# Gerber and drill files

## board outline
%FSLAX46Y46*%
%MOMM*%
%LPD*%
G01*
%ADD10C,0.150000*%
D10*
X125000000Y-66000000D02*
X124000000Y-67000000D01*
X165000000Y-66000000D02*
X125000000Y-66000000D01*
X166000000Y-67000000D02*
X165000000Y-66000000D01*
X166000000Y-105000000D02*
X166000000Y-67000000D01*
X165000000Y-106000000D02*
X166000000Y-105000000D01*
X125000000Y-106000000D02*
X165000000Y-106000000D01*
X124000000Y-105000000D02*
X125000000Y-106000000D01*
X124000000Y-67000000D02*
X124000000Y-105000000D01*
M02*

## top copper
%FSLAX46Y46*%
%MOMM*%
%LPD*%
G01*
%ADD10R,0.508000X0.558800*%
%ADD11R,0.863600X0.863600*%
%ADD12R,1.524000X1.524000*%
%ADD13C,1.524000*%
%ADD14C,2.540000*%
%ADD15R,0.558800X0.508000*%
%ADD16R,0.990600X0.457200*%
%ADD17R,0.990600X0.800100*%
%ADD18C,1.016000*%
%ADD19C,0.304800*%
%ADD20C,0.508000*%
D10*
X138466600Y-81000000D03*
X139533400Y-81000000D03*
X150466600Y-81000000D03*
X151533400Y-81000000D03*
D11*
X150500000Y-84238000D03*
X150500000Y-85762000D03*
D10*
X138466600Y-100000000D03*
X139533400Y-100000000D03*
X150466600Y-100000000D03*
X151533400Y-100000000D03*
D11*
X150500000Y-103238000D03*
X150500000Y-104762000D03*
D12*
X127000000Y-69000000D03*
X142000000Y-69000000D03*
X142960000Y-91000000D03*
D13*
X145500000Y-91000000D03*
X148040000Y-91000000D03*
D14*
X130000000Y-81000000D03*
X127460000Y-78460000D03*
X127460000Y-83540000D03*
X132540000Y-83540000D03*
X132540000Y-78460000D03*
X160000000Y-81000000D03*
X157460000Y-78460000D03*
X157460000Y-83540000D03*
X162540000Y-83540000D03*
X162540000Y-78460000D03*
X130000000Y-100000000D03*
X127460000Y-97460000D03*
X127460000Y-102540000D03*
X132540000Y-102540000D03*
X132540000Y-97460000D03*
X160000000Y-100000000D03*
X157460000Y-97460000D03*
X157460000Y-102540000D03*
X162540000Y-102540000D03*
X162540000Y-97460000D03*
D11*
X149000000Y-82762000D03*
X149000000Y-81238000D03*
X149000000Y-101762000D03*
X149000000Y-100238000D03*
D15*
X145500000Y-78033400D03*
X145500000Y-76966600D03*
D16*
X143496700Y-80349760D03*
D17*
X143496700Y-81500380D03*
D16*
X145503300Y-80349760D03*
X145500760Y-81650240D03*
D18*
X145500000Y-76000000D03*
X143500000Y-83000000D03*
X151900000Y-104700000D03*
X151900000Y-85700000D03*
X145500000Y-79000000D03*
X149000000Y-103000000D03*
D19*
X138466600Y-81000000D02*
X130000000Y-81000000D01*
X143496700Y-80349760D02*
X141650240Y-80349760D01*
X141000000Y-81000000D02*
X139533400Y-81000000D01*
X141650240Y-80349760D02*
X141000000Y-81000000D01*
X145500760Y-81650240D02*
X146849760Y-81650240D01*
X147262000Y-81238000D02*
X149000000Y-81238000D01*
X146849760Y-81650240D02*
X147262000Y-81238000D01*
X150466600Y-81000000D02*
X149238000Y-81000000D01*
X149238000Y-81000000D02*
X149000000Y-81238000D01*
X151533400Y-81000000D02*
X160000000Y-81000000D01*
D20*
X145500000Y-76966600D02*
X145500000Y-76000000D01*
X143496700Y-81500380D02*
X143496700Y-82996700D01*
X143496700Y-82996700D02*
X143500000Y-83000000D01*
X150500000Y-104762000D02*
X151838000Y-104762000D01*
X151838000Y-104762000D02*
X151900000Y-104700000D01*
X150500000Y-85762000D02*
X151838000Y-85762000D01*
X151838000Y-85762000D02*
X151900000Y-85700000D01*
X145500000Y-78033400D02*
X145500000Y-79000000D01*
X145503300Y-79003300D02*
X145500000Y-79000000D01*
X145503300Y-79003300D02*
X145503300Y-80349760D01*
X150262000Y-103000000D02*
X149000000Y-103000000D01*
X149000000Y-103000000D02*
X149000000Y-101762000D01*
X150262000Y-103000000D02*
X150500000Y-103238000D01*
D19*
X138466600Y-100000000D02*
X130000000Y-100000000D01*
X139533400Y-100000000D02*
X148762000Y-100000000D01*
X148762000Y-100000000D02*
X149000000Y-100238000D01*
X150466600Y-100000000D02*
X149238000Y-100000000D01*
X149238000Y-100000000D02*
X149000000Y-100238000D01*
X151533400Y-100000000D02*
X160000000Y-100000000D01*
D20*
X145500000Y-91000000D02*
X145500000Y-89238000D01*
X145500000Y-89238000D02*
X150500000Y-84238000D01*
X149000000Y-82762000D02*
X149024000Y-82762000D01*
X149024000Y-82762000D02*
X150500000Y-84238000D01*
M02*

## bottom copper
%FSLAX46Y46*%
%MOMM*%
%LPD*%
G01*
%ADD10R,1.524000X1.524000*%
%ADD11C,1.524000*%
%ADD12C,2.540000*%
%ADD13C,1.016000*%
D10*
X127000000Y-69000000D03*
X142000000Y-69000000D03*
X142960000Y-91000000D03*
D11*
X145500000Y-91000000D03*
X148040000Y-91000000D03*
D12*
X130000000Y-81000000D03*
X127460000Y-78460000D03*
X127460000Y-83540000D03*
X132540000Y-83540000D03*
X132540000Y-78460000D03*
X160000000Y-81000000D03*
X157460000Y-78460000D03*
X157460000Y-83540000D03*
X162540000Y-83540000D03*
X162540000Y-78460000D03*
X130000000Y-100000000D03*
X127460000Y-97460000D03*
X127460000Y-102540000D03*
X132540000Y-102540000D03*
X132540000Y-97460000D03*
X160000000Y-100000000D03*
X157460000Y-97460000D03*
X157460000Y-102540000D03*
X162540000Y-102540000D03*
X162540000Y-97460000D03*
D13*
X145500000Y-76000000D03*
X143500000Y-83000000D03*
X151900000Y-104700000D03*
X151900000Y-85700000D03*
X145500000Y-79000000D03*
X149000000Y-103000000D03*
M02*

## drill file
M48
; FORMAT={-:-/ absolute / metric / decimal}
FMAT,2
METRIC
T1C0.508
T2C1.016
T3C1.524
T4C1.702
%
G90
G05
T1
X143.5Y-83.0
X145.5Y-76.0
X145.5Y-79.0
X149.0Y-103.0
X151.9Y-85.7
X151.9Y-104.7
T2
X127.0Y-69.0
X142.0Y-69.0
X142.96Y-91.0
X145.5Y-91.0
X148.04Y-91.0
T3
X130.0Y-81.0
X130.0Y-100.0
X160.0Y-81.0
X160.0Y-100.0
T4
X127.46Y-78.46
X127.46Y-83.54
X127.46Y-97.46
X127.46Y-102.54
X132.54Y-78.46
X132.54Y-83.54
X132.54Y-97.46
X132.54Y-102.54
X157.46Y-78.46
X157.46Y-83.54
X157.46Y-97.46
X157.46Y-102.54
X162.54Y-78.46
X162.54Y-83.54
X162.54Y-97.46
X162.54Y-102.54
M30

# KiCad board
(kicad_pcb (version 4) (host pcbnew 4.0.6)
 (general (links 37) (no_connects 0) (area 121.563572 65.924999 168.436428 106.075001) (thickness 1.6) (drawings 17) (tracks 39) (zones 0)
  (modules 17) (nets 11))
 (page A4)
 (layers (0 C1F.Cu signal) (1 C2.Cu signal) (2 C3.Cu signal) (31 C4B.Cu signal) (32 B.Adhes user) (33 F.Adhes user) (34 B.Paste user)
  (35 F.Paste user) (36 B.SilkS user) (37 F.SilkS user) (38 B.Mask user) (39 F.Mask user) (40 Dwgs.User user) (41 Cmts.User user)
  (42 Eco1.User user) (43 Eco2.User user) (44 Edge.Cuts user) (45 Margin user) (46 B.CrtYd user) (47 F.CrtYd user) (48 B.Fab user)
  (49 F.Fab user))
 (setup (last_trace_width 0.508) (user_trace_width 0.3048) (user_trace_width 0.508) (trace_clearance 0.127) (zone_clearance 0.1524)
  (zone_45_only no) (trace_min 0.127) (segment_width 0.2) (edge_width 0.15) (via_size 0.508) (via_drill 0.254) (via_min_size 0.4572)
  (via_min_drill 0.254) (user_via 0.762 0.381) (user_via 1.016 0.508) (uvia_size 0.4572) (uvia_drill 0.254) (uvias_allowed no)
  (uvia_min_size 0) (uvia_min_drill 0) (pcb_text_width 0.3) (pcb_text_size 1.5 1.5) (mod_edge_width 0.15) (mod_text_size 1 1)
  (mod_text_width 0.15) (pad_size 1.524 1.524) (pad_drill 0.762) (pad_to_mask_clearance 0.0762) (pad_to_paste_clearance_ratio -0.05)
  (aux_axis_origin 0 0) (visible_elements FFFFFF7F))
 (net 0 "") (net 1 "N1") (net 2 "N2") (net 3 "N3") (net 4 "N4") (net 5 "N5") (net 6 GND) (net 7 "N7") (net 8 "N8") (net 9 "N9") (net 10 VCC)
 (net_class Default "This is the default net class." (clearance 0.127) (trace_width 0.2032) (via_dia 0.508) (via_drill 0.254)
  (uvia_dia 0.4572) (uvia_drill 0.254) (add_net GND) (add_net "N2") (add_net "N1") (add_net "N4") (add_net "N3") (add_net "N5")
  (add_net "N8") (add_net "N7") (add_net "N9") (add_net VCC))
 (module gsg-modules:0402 (layer C1F.Cu) (at 139 81 180) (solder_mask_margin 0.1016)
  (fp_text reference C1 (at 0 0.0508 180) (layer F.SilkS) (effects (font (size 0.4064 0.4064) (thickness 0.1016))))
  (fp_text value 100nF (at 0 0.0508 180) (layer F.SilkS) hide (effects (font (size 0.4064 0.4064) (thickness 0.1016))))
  (pad 2 smd rect (at 0.5334 0 180) (size 0.508 0.5588) (layers C1F.Cu F.Paste F.Mask) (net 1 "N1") (solder_mask_margin 0.1016))
  (pad 1 smd rect (at -0.5334 0 180) (size 0.508 0.5588) (layers C1F.Cu F.Paste F.Mask) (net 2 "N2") (solder_mask_margin 0.1016)))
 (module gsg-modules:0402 (layer C1F.Cu) (at 151 81 180) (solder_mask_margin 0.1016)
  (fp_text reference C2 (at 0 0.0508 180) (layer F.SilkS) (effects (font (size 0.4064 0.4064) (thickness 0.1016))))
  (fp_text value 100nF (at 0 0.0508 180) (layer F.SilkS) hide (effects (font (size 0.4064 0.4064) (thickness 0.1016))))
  (pad 2 smd rect (at 0.5334 0 180) (size 0.508 0.5588) (layers C1F.Cu F.Paste F.Mask) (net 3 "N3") (solder_mask_margin 0.1016))
  (pad 1 smd rect (at -0.5334 0 180) (size 0.508 0.5588) (layers C1F.Cu F.Paste F.Mask) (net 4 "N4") (solder_mask_margin 0.1016)))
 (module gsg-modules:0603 (layer C1F.Cu) (at 150.5 85 90) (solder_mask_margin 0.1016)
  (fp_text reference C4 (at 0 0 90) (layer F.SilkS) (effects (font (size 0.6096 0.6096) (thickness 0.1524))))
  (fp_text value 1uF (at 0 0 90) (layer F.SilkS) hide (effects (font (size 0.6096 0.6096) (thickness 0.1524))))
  (pad 2 smd rect (at 0.762 0 90) (size 0.8636 0.8636) (layers C1F.Cu F.Paste F.Mask) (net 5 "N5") (solder_mask_margin 0.1016)
   (clearance 0.1778))
  (pad 1 smd rect (at -0.762 0 90) (size 0.8636 0.8636) (layers C1F.Cu F.Paste F.Mask) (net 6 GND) (solder_mask_margin 0.1016)
   (clearance 0.1778)))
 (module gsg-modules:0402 (layer C1F.Cu) (at 139 100 180) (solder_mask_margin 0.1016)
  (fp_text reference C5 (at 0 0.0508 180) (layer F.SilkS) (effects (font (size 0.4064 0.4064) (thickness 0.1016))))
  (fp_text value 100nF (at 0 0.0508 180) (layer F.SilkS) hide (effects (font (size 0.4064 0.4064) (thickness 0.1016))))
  (pad 2 smd rect (at 0.5334 0 180) (size 0.508 0.5588) (layers C1F.Cu F.Paste F.Mask) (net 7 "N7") (solder_mask_margin 0.1016))
  (pad 1 smd rect (at -0.5334 0 180) (size 0.508 0.5588) (layers C1F.Cu F.Paste F.Mask) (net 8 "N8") (solder_mask_margin 0.1016)))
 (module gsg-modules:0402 (layer C1F.Cu) (at 151 100 180) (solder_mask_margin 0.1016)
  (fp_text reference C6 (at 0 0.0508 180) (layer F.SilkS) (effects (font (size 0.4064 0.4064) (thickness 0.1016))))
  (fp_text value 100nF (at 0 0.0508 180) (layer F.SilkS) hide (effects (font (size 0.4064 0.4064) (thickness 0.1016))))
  (pad 2 smd rect (at 0.5334 0 180) (size 0.508 0.5588) (layers C1F.Cu F.Paste F.Mask) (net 8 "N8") (solder_mask_margin 0.1016))
  (pad 1 smd rect (at -0.5334 0 180) (size 0.508 0.5588) (layers C1F.Cu F.Paste F.Mask) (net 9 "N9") (solder_mask_margin 0.1016)))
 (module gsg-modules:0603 (layer C1F.Cu) (at 150.5 104 90) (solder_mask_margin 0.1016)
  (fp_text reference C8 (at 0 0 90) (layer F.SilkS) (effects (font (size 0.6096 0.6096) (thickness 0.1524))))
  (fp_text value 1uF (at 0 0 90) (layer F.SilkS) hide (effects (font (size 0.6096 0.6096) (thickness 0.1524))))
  (pad 2 smd rect (at 0.762 0 90) (size 0.8636 0.8636) (layers C1F.Cu F.Paste F.Mask) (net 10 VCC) (solder_mask_margin 0.1016)
   (clearance 0.1778))
  (pad 1 smd rect (at -0.762 0 90) (size 0.8636 0.8636) (layers C1F.Cu F.Paste F.Mask) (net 6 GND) (solder_mask_margin 0.1016)
   (clearance 0.1778)))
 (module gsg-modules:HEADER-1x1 (layer C1F.Cu) (at 127 69)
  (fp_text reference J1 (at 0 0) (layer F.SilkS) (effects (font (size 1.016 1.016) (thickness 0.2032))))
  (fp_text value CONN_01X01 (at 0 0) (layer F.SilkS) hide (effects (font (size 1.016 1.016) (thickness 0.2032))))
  (pad 1 thru_hole rect (at 0 0) (size 1.524 1.524) (drill 1.016) (layers *.Cu *.Mask F.SilkS) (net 10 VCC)))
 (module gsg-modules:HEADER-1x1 (layer C1F.Cu) (at 142 69)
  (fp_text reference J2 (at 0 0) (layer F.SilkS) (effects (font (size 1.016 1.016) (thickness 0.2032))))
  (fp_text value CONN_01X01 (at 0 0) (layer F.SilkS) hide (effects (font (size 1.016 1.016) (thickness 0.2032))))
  (pad 1 thru_hole rect (at 0 0) (size 1.524 1.524) (drill 1.016) (layers *.Cu *.Mask F.SilkS) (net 6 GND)))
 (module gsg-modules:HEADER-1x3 (layer C1F.Cu) (at 145.5 91)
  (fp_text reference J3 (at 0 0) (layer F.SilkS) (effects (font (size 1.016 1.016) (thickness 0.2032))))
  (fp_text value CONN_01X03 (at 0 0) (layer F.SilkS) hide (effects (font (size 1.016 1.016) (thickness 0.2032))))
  (pad 1 thru_hole rect (at -2.54 0) (size 1.524 1.524) (drill 1.016) (layers *.Cu *.Mask F.SilkS) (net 10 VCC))
  (pad 2 thru_hole circle (at 0 0) (size 1.524 1.524) (drill 1.016) (layers *.Cu *.Mask F.SilkS) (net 5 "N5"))
  (pad 3 thru_hole circle (at 2.54 0) (size 1.524 1.524) (drill 1.016) (layers *.Cu *.Mask F.SilkS) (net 6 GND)))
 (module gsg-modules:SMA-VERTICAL (layer C1F.Cu) (at 130 81)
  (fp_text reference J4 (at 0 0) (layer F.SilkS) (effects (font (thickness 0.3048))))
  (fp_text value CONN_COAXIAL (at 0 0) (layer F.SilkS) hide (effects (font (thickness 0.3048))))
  (pad 1 thru_hole circle (at 0 0) (size 2.54 2.54) (drill 1.524) (layers *.Cu *.Mask F.SilkS) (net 1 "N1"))
  (pad 2 thru_hole circle (at -2.54 -2.54) (size 2.54 2.54) (drill 1.7018) (layers *.Cu *.Mask F.SilkS) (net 6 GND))
  (pad 2 thru_hole circle (at -2.54 2.54) (size 2.54 2.54) (drill 1.7018) (layers *.Cu *.Mask F.SilkS) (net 6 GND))
  (pad 2 thru_hole circle (at 2.54 2.54) (size 2.54 2.54) (drill 1.7018) (layers *.Cu *.Mask F.SilkS) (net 6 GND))
  (pad 2 thru_hole circle (at 2.54 -2.54) (size 2.54 2.54) (drill 1.7018) (layers *.Cu *.Mask F.SilkS) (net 6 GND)))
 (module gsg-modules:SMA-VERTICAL (layer C1F.Cu) (at 160 81)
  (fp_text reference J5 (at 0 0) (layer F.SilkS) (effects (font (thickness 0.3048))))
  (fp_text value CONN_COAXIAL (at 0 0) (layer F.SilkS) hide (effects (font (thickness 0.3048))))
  (pad 1 thru_hole circle (at 0 0) (size 2.54 2.54) (drill 1.524) (layers *.Cu *.Mask F.SilkS) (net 4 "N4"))
  (pad 2 thru_hole circle (at -2.54 -2.54) (size 2.54 2.54) (drill 1.7018) (layers *.Cu *.Mask F.SilkS) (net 6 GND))
  (pad 2 thru_hole circle (at -2.54 2.54) (size 2.54 2.54) (drill 1.7018) (layers *.Cu *.Mask F.SilkS) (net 6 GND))
  (pad 2 thru_hole circle (at 2.54 2.54) (size 2.54 2.54) (drill 1.7018) (layers *.Cu *.Mask F.SilkS) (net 6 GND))
  (pad 2 thru_hole circle (at 2.54 -2.54) (size 2.54 2.54) (drill 1.7018) (layers *.Cu *.Mask F.SilkS) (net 6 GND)))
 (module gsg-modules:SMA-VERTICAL (layer C1F.Cu) (at 130 100)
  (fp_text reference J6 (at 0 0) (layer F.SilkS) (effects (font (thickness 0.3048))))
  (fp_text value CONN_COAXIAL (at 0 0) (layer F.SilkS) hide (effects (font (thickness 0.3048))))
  (pad 1 thru_hole circle (at 0 0) (size 2.54 2.54) (drill 1.524) (layers *.Cu *.Mask F.SilkS) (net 7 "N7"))
  (pad 2 thru_hole circle (at -2.54 -2.54) (size 2.54 2.54) (drill 1.7018) (layers *.Cu *.Mask F.SilkS) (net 6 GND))
  (pad 2 thru_hole circle (at -2.54 2.54) (size 2.54 2.54) (drill 1.7018) (layers *.Cu *.Mask F.SilkS) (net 6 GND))
  (pad 2 thru_hole circle (at 2.54 2.54) (size 2.54 2.54) (drill 1.7018) (layers *.Cu *.Mask F.SilkS) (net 6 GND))
  (pad 2 thru_hole circle (at 2.54 -2.54) (size 2.54 2.54) (drill 1.7018) (layers *.Cu *.Mask F.SilkS) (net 6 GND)))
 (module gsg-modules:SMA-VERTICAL (layer C1F.Cu) (at 160 100)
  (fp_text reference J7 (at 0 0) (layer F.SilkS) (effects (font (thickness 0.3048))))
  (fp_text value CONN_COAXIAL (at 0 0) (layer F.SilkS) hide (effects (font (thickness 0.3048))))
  (pad 1 thru_hole circle (at 0 0) (size 2.54 2.54) (drill 1.524) (layers *.Cu *.Mask F.SilkS) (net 9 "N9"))
  (pad 2 thru_hole circle (at -2.54 -2.54) (size 2.54 2.54) (drill 1.7018) (layers *.Cu *.Mask F.SilkS) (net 6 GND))
  (pad 2 thru_hole circle (at -2.54 2.54) (size 2.54 2.54) (drill 1.7018) (layers *.Cu *.Mask F.SilkS) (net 6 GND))
  (pad 2 thru_hole circle (at 2.54 2.54) (size 2.54 2.54) (drill 1.7018) (layers *.Cu *.Mask F.SilkS) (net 6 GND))
  (pad 2 thru_hole circle (at 2.54 -2.54) (size 2.54 2.54) (drill 1.7018) (layers *.Cu *.Mask F.SilkS) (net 6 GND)))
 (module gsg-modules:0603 (layer C1F.Cu) (at 149 82 270) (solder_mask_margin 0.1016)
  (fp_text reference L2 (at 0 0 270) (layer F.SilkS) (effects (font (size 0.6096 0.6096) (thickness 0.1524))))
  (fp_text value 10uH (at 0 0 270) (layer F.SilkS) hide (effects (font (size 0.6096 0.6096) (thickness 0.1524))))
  (pad 2 smd rect (at 0.762 0 270) (size 0.8636 0.8636) (layers C1F.Cu F.Paste F.Mask) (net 5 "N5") (solder_mask_margin 0.1016)
   (clearance 0.1778))
  (pad 1 smd rect (at -0.762 0 270) (size 0.8636 0.8636) (layers C1F.Cu F.Paste F.Mask) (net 3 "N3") (solder_mask_margin 0.1016)
   (clearance 0.1778)))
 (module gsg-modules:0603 (layer C1F.Cu) (at 149 101 270) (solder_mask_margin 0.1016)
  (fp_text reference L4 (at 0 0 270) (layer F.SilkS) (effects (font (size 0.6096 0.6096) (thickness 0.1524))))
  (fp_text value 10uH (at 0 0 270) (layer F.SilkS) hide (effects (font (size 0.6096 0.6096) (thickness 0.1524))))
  (pad 2 smd rect (at 0.762 0 270) (size 0.8636 0.8636) (layers C1F.Cu F.Paste F.Mask) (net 10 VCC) (solder_mask_margin 0.1016)
   (clearance 0.1778))
  (pad 1 smd rect (at -0.762 0 270) (size 0.8636 0.8636) (layers C1F.Cu F.Paste F.Mask) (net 8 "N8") (solder_mask_margin 0.1016)
   (clearance 0.1778)))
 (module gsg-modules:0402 (layer C1F.Cu) (at 145.5 77.5 270) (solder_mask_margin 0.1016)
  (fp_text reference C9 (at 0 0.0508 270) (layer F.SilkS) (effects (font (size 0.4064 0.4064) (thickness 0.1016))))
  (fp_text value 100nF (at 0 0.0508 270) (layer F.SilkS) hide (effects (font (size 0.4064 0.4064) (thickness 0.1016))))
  (pad 2 smd rect (at 0.5334 0 270) (size 0.508 0.5588) (layers C1F.Cu F.Paste F.Mask) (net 10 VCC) (solder_mask_margin 0.1016))
  (pad 1 smd rect (at -0.5334 0 270) (size 0.508 0.5588) (layers C1F.Cu F.Paste F.Mask) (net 6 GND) (solder_mask_margin 0.1016)))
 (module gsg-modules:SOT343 (layer C1F.Cu) (at 144.5 81 270)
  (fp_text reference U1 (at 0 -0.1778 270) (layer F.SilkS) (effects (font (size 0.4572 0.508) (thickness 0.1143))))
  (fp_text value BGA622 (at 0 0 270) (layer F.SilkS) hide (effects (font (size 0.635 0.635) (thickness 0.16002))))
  (pad 1 smd rect (at -0.65024 1.0033 270) (size 0.4572 0.9906) (layers C1F.Cu F.Paste F.Mask) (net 2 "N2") (die_length 0.08382))
  (pad 2 smd rect (at 0.50038 1.0033 270) (size 0.8001 0.9906) (layers C1F.Cu F.Paste F.Mask) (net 6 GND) (die_length -2147.483648))
  (pad 4 smd rect (at -0.65024 -1.0033 270) (size 0.4572 0.9906) (layers C1F.Cu F.Paste F.Mask) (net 10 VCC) (die_length -2147.483648))
  (pad 3 smd rect (at 0.65024 -1.00076 270) (size 0.4572 0.9906) (layers C1F.Cu F.Paste F.Mask) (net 3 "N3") (die_length 0.12192)))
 (gr_line (start 125 66) (end 124 67) (angle 90) (layer Edge.Cuts) (width 0.15))
 (gr_line (start 165 66) (end 125 66) (angle 90) (layer Edge.Cuts) (width 0.15))
 (gr_line (start 166 67) (end 165 66) (angle 90) (layer Edge.Cuts) (width 0.15))
 (gr_line (start 166 105) (end 166 67) (angle 90) (layer Edge.Cuts) (width 0.15))
 (gr_line (start 165 106) (end 166 105) (angle 90) (layer Edge.Cuts) (width 0.15))
 (gr_line (start 125 106) (end 165 106) (angle 90) (layer Edge.Cuts) (width 0.15))
 (gr_line (start 124 105) (end 125 106) (angle 90) (layer Edge.Cuts) (width 0.15))
 (gr_line (start 124 67) (end 124 105) (angle 90) (layer Edge.Cuts) (width 0.15))
 (segment (start 138.4666 81) (end 130 81) (width 0.3048) (layer C1F.Cu) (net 1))
 (segment (start 143.4967 80.34976) (end 141.65024 80.34976) (width 0.3048) (layer C1F.Cu) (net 2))
 (segment (start 141 81) (end 139.5334 81) (width 0.3048) (layer C1F.Cu) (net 2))
 (segment (start 141.65024 80.34976) (end 141 81) (width 0.3048) (layer C1F.Cu) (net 2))
 (segment (start 145.50076 81.65024) (end 146.84976 81.65024) (width 0.3048) (layer C1F.Cu) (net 3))
 (segment (start 147.262 81.238) (end 149 81.238) (width 0.3048) (layer C1F.Cu) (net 3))
 (segment (start 146.84976 81.65024) (end 147.262 81.238) (width 0.3048) (layer C1F.Cu) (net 3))
 (segment (start 150.4666 81) (end 149.238 81) (width 0.3048) (layer C1F.Cu) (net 3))
 (segment (start 149.238 81) (end 149 81.238) (width 0.3048) (layer C1F.Cu) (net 3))
 (segment (start 151.5334 81) (end 160 81) (width 0.3048) (layer C1F.Cu) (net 4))
 (segment (start 145.5 76.9666) (end 145.5 76) (width 0.508) (layer C1F.Cu) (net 6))
 (via (at 145.5 76) (size 1.016) (drill 0.508) (layers C1F.Cu C4B.Cu) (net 6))
 (segment (start 143.4967 81.50038) (end 143.4967 82.9967) (width 0.508) (layer C1F.Cu) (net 6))
 (via (at 143.5 83) (size 1.016) (drill 0.508) (layers C1F.Cu C4B.Cu) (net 6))
 (segment (start 143.4967 82.9967) (end 143.5 83) (width 0.508) (layer C1F.Cu) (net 6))
 (segment (start 150.5 104.762) (end 151.838 104.762) (width 0.508) (layer C1F.Cu) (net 6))
 (via (at 151.9 104.7) (size 1.016) (drill 0.508) (layers C1F.Cu C4B.Cu) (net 6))
 (segment (start 151.838 104.762) (end 151.9 104.7) (width 0.508) (layer C1F.Cu) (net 6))
 (segment (start 150.5 85.762) (end 151.838 85.762) (width 0.508) (layer C1F.Cu) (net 6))
 (via (at 151.9 85.7) (size 1.016) (drill 0.508) (layers C1F.Cu C4B.Cu) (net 6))
 (segment (start 151.838 85.762) (end 151.9 85.7) (width 0.508) (layer C1F.Cu) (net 6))
 (segment (start 145.5 78.0334) (end 145.5 79) (width 0.508) (layer C1F.Cu) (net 10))
 (segment (start 145.5033 79.0033) (end 145.5 79) (width 0.508) (layer C1F.Cu) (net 10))
 (via (at 145.5 79) (size 1.016) (drill 0.508) (layers C1F.Cu C4B.Cu) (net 10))
 (segment (start 145.5033 79.0033) (end 145.5033 80.34976) (width 0.508) (layer C1F.Cu) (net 10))
 (segment (start 150.262 103) (end 149 103) (width 0.508) (layer C1F.Cu) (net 10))
 (via (at 149 103) (size 1.016) (drill 0.508) (layers C1F.Cu C4B.Cu) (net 10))
 (segment (start 149 103) (end 149 101.762) (width 0.508) (layer C1F.Cu) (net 10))
 (segment (start 150.262 103) (end 150.5 103.238) (width 0.508) (layer C1F.Cu) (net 10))
 (segment (start 138.4666 100) (end 130 100) (width 0.3048) (layer C1F.Cu) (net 7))
 (segment (start 139.5334 100) (end 148.762 100) (width 0.3048) (layer C1F.Cu) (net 8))
 (segment (start 148.762 100) (end 149 100.238) (width 0.3048) (layer C1F.Cu) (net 8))
 (segment (start 150.4666 100) (end 149.238 100) (width 0.3048) (layer C1F.Cu) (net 8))
 (segment (start 149.238 100) (end 149 100.238) (width 0.3048) (layer C1F.Cu) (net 8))
 (segment (start 151.5334 100) (end 160 100) (width 0.3048) (layer C1F.Cu) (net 9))
 (segment (start 145.5 91) (end 145.5 89.238) (width 0.508) (layer C1F.Cu) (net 5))
 (segment (start 145.5 89.238) (end 150.5 84.238) (width 0.508) (layer C1F.Cu) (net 5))
 (segment (start 149 82.762) (end 149.024 82.762) (width 0.508) (layer C1F.Cu) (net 5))
 (segment (start 149.024 82.762) (end 150.5 84.238) (width 0.508) (layer C1F.Cu) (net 5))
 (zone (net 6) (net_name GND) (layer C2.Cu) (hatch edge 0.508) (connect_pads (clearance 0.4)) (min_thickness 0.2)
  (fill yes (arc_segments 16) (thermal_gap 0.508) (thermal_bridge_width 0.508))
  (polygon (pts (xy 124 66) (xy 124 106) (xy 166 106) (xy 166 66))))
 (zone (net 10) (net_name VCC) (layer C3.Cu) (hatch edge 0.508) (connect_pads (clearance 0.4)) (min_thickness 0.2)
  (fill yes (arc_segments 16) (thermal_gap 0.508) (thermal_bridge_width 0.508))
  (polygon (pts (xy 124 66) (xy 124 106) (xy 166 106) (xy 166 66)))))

